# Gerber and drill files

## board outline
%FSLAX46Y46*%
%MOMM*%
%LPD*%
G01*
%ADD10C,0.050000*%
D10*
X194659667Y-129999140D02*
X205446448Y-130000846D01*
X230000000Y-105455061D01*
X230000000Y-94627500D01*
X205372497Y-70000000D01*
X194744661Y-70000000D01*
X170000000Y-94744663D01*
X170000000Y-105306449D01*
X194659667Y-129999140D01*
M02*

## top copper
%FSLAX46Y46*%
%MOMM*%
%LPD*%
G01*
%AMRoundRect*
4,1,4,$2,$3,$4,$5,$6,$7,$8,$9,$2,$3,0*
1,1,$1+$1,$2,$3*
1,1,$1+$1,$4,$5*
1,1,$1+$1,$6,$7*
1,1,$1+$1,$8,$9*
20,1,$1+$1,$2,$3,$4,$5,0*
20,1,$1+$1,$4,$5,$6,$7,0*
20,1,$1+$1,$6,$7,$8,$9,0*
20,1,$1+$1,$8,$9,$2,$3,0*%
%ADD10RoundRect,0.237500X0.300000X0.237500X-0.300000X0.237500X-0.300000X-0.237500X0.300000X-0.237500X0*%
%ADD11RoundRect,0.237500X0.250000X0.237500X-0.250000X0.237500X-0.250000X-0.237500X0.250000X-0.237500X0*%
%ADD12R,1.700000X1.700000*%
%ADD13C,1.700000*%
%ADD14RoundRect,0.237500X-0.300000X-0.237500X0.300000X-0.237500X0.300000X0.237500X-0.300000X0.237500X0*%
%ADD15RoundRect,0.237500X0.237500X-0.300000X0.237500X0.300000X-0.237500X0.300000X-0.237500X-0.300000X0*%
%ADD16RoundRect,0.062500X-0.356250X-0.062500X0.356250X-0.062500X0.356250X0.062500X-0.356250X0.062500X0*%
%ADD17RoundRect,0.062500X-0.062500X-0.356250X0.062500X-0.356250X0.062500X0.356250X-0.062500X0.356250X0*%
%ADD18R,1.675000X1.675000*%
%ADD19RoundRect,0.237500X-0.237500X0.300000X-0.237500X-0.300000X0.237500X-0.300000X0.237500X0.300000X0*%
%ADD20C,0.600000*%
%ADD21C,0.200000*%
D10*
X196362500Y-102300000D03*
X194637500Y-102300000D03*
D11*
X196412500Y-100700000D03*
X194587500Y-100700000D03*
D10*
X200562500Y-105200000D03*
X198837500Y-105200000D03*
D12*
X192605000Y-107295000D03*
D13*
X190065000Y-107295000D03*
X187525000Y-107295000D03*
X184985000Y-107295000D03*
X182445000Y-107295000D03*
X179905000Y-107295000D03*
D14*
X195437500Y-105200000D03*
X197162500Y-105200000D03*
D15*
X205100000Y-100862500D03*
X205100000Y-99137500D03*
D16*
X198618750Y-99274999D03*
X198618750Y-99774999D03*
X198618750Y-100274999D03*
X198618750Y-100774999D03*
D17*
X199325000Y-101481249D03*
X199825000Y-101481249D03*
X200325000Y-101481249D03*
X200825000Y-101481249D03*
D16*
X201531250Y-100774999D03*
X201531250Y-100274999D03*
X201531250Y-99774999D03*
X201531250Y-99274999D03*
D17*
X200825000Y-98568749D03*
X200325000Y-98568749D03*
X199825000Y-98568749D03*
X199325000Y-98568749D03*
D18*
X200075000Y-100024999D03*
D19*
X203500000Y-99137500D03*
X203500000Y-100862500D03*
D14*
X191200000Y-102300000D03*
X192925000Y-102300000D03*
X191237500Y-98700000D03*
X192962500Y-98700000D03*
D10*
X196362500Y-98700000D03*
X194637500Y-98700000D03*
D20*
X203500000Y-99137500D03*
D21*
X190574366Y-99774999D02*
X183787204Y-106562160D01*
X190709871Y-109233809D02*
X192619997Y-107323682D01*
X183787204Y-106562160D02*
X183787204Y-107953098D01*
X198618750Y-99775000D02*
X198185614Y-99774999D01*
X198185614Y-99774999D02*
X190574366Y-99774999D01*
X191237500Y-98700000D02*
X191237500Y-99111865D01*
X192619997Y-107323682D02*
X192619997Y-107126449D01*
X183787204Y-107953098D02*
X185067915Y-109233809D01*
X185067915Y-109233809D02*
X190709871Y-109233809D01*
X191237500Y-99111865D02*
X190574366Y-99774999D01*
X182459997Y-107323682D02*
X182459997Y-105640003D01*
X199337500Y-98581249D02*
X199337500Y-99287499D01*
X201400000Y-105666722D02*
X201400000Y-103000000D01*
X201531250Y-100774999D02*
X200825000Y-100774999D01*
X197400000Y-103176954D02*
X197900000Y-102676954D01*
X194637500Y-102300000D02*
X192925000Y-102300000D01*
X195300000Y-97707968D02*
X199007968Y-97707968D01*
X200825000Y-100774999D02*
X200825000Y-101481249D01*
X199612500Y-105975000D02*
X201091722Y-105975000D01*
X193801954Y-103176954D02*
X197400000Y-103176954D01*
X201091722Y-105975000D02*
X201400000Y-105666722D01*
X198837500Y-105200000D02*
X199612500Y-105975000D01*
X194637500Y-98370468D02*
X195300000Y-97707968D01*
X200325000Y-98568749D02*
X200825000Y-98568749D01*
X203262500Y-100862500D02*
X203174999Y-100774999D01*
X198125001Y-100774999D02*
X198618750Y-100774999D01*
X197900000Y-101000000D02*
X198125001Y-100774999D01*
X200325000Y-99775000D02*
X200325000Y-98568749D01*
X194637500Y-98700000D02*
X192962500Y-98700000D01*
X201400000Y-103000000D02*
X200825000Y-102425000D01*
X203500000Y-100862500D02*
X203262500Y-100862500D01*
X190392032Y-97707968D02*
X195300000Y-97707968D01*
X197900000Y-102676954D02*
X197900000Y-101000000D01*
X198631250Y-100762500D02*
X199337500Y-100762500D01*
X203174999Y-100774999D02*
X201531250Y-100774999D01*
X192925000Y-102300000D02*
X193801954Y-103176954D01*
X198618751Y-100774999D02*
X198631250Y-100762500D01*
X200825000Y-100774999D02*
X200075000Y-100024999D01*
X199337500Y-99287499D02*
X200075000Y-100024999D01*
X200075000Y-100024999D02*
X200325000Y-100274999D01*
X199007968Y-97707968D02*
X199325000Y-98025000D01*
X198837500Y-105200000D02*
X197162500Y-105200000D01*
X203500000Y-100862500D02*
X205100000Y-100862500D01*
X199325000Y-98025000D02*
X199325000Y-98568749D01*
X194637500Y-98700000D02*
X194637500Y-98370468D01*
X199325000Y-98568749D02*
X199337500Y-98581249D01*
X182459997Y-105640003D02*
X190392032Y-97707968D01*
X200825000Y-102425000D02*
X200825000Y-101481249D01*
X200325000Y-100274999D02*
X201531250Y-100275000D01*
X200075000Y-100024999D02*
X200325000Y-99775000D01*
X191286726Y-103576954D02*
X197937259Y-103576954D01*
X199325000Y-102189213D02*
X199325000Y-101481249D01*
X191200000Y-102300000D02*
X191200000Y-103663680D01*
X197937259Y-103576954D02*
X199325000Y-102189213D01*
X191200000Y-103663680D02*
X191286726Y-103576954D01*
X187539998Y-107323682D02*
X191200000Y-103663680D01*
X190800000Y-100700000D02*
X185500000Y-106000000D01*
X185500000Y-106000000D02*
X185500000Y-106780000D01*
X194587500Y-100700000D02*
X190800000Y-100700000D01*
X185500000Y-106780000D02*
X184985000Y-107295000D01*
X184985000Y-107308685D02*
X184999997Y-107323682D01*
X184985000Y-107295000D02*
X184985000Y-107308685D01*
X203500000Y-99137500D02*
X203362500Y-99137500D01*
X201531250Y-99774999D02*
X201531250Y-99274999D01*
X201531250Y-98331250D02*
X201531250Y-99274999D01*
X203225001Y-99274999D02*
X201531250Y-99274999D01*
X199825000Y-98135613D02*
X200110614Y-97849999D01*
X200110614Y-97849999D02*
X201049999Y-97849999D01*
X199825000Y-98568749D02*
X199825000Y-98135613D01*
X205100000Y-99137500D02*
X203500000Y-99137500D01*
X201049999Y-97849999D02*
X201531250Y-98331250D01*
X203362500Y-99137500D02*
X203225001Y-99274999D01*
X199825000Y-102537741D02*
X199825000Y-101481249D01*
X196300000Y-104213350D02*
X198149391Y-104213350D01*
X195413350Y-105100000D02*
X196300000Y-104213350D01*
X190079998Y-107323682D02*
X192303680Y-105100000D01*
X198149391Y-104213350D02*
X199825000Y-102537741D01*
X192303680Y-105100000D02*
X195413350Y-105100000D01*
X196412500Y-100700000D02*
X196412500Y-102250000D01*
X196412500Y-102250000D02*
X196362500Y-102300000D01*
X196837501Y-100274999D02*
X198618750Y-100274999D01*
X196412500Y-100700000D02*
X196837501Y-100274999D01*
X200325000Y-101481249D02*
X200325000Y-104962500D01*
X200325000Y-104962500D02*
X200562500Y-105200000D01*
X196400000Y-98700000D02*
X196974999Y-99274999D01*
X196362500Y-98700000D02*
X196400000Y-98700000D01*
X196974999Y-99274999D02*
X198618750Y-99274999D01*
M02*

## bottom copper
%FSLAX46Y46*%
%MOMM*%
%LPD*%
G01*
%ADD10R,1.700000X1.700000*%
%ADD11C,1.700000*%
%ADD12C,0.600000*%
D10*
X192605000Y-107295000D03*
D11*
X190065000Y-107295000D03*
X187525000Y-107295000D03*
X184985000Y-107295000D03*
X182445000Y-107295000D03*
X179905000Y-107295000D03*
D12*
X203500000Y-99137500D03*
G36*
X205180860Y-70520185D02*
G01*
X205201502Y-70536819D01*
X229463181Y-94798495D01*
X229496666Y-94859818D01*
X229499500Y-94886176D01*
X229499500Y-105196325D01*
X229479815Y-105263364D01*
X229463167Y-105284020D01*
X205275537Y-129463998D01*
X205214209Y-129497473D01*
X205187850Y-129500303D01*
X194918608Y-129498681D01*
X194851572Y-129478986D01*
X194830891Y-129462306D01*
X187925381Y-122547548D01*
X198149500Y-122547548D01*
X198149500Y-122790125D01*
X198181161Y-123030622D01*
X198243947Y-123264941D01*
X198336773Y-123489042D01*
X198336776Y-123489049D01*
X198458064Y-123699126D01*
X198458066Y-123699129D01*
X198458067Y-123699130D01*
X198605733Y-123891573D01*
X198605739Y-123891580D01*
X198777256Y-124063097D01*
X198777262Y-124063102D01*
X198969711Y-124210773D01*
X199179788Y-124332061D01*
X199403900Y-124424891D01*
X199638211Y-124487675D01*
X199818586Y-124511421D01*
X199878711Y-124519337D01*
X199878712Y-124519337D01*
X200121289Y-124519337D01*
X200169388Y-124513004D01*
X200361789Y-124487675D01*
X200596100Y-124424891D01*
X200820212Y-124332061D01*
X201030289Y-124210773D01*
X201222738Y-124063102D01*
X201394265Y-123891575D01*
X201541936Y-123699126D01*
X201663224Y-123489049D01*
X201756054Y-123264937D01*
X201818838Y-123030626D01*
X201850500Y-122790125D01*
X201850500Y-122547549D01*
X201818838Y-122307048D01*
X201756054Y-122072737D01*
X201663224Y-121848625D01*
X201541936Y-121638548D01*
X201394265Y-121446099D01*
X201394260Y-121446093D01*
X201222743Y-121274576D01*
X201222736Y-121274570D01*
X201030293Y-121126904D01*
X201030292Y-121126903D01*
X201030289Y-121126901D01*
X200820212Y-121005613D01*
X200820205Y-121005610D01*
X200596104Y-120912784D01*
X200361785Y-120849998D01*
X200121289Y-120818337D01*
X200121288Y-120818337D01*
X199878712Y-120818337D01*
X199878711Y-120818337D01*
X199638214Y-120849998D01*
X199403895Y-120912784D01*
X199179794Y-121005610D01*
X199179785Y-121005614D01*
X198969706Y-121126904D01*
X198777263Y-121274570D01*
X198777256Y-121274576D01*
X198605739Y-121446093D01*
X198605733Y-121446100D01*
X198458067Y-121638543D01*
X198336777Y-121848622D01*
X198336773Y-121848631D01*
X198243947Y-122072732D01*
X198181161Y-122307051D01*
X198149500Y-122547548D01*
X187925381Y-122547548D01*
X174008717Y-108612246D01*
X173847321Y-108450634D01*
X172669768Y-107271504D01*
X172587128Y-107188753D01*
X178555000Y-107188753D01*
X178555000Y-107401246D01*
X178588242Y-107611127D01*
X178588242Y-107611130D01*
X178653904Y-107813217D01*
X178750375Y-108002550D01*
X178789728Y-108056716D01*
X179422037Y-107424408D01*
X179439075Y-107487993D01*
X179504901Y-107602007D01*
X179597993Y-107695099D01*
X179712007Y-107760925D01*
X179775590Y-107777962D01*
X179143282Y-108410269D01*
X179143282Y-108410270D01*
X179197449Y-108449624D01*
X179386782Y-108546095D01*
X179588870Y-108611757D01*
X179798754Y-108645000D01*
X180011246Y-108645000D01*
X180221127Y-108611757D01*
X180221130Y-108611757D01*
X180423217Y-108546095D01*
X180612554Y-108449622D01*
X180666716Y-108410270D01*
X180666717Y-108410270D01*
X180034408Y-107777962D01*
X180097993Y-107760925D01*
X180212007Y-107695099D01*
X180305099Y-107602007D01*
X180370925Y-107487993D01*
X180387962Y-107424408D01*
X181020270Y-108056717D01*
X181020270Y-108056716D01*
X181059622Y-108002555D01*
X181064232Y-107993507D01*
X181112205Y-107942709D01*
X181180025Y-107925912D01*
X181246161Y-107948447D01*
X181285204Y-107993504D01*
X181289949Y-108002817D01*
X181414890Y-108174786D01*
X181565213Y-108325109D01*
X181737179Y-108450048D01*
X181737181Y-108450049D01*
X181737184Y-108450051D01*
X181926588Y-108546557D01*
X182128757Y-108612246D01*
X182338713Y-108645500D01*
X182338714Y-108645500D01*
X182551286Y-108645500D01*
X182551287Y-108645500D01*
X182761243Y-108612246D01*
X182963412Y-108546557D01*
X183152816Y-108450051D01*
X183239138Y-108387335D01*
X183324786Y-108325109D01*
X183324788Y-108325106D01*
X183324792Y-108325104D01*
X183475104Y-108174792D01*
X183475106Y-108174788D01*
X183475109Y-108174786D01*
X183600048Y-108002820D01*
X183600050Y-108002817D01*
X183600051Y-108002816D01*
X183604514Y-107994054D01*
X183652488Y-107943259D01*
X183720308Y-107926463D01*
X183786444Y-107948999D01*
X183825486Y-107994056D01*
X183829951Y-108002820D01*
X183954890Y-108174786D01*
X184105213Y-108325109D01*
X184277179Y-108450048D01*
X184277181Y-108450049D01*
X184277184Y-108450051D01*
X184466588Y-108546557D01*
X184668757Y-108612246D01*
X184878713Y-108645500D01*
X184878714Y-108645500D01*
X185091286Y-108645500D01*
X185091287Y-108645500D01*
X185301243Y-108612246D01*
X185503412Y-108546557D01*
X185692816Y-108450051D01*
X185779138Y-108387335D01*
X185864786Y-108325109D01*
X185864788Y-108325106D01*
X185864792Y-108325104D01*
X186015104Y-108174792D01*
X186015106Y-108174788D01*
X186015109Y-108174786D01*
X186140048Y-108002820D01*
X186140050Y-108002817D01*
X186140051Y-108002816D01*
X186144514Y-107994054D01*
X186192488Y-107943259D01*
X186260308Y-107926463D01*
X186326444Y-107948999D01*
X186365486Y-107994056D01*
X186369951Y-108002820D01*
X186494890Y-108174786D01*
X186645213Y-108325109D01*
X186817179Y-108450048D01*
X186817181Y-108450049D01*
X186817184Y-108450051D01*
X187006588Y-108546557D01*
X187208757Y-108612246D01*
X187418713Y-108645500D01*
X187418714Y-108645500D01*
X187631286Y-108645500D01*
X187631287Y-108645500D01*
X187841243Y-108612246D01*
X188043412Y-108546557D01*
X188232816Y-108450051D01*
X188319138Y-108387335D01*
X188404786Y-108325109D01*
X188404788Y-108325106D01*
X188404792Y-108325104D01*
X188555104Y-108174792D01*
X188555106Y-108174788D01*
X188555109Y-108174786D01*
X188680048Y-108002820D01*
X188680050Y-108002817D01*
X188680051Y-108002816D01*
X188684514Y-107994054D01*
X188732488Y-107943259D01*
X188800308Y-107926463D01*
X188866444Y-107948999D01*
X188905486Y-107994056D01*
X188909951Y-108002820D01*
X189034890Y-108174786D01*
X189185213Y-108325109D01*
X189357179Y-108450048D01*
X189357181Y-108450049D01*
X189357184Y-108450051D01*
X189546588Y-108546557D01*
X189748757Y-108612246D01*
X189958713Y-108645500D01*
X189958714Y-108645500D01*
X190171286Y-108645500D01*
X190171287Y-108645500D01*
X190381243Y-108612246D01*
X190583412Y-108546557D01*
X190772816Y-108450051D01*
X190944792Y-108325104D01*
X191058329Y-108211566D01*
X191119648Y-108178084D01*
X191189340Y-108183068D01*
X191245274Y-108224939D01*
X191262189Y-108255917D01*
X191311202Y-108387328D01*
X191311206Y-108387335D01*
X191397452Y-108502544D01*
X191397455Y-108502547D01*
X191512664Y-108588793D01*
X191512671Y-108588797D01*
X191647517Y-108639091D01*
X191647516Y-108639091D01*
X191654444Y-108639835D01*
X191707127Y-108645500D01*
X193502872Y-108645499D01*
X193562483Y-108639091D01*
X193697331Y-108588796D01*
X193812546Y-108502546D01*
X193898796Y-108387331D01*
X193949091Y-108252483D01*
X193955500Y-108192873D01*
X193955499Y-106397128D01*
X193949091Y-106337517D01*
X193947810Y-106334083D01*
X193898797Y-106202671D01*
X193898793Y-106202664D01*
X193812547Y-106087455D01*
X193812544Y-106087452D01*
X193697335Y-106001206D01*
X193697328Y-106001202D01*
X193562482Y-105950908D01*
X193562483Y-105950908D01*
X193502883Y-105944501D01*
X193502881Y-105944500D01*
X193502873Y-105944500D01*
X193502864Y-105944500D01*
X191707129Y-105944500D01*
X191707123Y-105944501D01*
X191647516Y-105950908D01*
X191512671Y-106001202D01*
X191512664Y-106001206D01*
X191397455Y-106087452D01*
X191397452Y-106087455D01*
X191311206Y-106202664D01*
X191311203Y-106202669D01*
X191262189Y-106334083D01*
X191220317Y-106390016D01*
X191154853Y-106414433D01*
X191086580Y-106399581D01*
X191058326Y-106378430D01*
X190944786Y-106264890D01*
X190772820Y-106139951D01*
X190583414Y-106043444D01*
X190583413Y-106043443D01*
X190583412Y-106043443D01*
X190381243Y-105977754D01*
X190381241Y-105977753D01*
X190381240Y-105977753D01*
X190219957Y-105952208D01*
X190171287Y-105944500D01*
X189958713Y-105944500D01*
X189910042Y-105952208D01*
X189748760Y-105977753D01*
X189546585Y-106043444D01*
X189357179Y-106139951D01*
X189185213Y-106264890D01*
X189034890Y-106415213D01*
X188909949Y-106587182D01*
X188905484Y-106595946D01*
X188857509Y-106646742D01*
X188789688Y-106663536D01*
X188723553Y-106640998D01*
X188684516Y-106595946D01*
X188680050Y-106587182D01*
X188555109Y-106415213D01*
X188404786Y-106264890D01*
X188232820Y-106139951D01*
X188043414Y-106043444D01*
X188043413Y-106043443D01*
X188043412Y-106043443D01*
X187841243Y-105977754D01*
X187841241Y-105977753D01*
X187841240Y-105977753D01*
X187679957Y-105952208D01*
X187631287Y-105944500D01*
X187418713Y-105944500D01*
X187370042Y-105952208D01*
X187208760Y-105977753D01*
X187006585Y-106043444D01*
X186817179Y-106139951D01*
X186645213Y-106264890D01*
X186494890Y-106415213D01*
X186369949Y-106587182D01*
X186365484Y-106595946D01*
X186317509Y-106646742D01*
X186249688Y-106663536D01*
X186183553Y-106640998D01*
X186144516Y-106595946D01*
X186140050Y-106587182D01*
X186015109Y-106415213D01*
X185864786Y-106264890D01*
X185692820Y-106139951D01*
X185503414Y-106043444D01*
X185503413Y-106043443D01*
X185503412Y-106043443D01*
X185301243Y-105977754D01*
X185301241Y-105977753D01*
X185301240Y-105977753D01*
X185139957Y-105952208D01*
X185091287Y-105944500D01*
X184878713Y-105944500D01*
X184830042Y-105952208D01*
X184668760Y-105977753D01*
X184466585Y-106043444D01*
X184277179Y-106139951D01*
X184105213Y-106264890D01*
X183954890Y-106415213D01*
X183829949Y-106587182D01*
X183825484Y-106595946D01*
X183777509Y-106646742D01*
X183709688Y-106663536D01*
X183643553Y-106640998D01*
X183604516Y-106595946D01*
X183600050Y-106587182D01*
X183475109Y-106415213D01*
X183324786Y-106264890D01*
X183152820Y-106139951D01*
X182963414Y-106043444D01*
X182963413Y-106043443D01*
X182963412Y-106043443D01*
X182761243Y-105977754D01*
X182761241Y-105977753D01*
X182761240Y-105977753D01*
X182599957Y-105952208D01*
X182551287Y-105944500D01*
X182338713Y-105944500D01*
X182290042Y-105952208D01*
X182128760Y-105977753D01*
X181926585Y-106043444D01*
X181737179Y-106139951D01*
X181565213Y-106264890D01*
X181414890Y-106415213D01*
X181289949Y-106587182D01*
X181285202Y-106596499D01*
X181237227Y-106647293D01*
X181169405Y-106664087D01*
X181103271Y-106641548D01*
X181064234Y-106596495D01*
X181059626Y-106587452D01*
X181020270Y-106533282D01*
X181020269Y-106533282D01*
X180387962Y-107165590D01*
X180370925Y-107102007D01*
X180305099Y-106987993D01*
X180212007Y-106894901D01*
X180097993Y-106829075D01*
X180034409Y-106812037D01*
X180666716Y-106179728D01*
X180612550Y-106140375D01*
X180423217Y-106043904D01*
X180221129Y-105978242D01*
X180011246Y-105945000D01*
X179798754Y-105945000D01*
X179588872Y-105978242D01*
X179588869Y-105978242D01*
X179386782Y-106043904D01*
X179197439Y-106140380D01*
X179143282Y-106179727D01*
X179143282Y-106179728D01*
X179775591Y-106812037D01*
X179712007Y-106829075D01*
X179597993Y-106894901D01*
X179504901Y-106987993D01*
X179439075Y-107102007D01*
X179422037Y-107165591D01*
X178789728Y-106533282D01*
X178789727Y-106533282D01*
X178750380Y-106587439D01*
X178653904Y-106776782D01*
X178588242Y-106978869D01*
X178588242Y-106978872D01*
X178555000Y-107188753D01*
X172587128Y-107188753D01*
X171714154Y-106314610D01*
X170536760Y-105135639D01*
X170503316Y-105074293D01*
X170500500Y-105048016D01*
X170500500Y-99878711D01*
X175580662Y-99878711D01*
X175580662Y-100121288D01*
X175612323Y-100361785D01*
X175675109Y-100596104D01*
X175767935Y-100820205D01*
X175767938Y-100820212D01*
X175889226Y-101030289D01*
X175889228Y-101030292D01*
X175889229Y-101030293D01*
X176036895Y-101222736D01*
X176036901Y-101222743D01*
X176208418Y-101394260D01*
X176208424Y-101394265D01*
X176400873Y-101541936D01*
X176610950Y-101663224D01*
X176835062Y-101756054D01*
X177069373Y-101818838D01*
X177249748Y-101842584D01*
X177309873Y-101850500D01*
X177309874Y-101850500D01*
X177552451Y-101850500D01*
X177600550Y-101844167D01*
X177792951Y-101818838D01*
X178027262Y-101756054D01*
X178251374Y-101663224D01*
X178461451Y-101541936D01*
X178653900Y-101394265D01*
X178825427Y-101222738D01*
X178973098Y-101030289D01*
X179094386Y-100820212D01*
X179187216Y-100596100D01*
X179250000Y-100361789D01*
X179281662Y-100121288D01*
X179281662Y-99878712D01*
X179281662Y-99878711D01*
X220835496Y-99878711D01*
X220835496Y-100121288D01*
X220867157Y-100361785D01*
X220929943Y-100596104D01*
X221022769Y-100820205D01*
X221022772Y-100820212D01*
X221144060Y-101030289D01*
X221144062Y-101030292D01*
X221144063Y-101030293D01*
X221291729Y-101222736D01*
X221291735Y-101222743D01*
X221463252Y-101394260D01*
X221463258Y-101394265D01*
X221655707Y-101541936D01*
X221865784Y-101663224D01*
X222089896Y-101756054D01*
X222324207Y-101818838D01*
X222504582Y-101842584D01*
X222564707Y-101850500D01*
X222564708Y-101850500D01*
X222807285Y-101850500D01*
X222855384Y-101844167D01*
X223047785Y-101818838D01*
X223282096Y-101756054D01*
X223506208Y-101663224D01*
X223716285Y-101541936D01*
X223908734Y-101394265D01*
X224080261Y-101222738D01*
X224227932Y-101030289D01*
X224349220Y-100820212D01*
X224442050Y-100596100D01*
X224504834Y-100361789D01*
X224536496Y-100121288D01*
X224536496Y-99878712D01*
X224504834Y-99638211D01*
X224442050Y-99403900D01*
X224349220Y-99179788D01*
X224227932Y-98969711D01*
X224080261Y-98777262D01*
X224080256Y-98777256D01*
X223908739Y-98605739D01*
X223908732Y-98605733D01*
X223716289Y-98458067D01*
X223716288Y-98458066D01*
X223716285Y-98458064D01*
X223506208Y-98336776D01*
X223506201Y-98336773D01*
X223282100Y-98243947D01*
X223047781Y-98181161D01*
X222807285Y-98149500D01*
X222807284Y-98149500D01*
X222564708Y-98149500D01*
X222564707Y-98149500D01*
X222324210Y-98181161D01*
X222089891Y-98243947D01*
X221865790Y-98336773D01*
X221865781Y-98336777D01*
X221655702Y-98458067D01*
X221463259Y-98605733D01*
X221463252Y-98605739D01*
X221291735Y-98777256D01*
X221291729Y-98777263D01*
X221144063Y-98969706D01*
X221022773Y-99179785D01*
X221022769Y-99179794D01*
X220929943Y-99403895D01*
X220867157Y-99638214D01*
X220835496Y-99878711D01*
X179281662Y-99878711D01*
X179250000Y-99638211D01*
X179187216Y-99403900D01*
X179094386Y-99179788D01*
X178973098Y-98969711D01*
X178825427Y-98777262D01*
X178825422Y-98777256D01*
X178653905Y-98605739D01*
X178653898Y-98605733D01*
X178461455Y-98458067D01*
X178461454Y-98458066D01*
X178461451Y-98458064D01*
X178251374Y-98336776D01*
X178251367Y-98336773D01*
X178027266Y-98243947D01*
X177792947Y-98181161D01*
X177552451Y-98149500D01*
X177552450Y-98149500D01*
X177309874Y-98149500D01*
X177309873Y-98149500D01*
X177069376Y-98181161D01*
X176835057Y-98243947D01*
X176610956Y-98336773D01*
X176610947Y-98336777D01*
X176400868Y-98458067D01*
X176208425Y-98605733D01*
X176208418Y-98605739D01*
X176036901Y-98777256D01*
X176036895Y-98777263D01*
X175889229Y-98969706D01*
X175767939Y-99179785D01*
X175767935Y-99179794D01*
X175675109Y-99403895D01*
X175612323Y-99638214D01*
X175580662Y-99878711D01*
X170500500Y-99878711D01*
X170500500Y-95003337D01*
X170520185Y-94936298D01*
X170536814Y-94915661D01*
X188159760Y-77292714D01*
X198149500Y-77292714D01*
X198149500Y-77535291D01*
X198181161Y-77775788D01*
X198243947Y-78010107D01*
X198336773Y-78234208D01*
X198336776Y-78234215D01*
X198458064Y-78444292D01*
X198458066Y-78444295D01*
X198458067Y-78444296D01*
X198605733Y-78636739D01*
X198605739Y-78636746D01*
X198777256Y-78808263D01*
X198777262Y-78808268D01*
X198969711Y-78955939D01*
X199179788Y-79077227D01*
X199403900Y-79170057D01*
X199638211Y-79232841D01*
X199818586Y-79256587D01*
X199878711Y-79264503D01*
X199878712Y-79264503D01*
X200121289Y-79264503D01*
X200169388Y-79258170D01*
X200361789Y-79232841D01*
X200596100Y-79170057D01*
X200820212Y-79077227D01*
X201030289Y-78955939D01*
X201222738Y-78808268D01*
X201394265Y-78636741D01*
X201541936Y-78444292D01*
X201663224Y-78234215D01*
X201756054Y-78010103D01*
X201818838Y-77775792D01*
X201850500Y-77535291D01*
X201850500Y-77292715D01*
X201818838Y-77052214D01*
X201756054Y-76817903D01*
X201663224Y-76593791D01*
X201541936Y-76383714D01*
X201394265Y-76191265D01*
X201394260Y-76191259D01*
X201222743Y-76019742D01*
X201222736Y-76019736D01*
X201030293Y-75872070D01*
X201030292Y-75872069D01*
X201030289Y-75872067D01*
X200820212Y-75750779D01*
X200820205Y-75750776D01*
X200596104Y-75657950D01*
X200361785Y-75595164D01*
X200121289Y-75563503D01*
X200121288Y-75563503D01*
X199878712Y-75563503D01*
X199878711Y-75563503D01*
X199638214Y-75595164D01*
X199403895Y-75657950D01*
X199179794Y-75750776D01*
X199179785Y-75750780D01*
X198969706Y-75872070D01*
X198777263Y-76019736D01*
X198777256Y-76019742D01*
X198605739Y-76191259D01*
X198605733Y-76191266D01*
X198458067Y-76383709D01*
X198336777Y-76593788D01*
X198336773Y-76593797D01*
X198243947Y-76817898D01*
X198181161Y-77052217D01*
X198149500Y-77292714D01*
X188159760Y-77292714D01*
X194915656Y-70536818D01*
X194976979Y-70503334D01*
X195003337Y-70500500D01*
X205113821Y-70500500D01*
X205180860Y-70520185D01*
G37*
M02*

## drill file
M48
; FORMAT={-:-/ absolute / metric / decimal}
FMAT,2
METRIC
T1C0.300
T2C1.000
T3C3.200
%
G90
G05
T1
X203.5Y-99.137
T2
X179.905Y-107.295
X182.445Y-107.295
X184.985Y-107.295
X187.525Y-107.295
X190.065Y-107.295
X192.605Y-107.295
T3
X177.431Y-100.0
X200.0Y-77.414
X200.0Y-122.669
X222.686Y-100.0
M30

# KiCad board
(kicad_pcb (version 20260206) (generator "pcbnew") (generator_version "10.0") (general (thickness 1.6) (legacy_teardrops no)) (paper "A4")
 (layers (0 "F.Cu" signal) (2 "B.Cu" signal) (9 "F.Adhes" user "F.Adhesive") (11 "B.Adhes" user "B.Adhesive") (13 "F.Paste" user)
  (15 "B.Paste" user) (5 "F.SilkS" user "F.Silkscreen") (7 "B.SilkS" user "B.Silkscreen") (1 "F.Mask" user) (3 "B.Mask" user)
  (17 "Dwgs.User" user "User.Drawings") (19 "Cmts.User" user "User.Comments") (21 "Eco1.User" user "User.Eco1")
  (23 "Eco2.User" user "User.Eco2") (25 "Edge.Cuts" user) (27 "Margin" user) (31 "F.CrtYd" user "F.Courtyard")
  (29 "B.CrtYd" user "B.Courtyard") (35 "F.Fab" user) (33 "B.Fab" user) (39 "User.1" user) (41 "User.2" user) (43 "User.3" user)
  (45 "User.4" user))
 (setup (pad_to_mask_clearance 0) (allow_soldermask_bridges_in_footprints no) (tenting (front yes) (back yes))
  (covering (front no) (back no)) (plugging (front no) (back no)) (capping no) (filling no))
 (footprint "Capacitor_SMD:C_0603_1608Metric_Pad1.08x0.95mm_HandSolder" (layer "F.Cu") (at 195.5 102.3 180)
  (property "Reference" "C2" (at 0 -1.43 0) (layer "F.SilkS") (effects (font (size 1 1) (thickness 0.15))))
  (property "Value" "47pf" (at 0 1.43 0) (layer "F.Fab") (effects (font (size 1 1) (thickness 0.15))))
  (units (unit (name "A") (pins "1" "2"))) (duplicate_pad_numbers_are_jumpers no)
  (pad "1" smd roundrect (at -0.8625 0 180) (size 1.075 0.95) (layers "F.Cu" "F.Mask" "F.Paste") (roundrect_rratio 0.25)
   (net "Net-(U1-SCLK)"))
  (pad "2" smd roundrect (at 0.8625 0 180) (size 1.075 0.95) (layers "F.Cu" "F.Mask" "F.Paste") (roundrect_rratio 0.25) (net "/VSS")))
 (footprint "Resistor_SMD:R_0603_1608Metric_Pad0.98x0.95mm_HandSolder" (layer "F.Cu") (at 195.5 100.7 180)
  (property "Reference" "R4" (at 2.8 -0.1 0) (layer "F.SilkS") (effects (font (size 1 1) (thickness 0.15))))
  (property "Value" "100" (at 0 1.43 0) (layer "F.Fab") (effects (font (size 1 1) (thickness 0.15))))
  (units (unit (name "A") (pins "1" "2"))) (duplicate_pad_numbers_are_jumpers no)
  (pad "1" smd roundrect (at -0.9125 0 180) (size 0.975 0.95) (layers "F.Cu" "F.Mask" "F.Paste") (roundrect_rratio 0.25)
   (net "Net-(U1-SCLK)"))
  (pad "2" smd roundrect (at 0.9125 0 180) (size 0.975 0.95) (layers "F.Cu" "F.Mask" "F.Paste") (roundrect_rratio 0.25) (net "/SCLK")))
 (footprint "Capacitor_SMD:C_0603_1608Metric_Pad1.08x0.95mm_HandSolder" (layer "F.Cu") (at 199.7 105.2 180)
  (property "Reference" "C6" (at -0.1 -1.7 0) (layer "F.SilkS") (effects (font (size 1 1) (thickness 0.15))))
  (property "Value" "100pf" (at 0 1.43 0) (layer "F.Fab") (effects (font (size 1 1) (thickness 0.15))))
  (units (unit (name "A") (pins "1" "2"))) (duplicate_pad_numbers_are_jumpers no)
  (pad "1" smd roundrect (at -0.8625 0 180) (size 1.075 0.95) (layers "F.Cu" "F.Mask" "F.Paste") (roundrect_rratio 0.25)
   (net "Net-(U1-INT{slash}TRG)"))
  (pad "2" smd roundrect (at 0.8625 0 180) (size 1.075 0.95) (layers "F.Cu" "F.Mask" "F.Paste") (roundrect_rratio 0.25) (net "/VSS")))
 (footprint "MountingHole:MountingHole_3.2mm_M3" (layer "F.Cu") (at 200 77.414003 45)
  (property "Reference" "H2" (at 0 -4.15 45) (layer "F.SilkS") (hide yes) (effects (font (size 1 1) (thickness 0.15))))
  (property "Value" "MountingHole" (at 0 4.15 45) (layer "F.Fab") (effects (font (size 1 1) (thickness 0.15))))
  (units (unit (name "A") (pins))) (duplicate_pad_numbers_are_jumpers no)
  (pad "" np_thru_hole circle (at 0 0 45) (size 3.2 3.2) (drill 3.2) (layers "*.Cu" "*.Mask")))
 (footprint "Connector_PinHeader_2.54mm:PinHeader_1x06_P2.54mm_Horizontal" (layer "F.Cu") (at 192.605 107.295 -90)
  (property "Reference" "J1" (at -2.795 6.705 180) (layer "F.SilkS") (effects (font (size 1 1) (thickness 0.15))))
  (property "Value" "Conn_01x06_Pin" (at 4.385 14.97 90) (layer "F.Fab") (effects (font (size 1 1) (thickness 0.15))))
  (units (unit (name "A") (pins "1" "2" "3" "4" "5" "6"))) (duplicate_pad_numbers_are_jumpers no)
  (pad "1" thru_hole rect (at 0 0 270) (size 1.7 1.7) (drill 1) (layers "*.Cu" "*.Mask") (remove_unused_layers no) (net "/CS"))
  (pad "2" thru_hole circle (at 0 2.54 270) (size 1.7 1.7) (drill 1) (layers "*.Cu" "*.Mask") (remove_unused_layers no) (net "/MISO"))
  (pad "3" thru_hole circle (at 0 5.08 270) (size 1.7 1.7) (drill 1) (layers "*.Cu" "*.Mask") (remove_unused_layers no) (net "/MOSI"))
  (pad "4" thru_hole circle (at 0 7.62 270) (size 1.7 1.7) (drill 1) (layers "*.Cu" "*.Mask") (remove_unused_layers no) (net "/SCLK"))
  (pad "5" thru_hole circle (at 0 10.16 270) (size 1.7 1.7) (drill 1) (layers "*.Cu" "*.Mask") (remove_unused_layers no) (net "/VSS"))
  (pad "6" thru_hole circle (at 0 12.7 270) (size 1.7 1.7) (drill 1) (layers "*.Cu" "*.Mask") (remove_unused_layers no) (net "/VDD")))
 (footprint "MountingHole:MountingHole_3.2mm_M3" (layer "F.Cu") (at 200 122.668837 45)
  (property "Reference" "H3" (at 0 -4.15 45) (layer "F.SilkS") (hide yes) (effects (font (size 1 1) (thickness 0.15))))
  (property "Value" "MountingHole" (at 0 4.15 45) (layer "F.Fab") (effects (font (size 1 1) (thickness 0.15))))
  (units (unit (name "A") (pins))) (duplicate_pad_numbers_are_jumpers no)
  (pad "" np_thru_hole circle (at 0 0 45) (size 3.2 3.2) (drill 3.2) (layers "*.Cu" "*.Mask")))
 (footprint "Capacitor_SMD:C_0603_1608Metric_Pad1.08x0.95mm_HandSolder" (layer "F.Cu") (at 196.3 105.2)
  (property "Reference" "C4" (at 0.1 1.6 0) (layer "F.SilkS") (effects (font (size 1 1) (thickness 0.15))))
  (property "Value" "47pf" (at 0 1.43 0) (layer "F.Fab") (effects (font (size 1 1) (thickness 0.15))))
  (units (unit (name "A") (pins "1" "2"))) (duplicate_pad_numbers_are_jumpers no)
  (pad "1" smd roundrect (at -0.8625 0) (size 1.075 0.95) (layers "F.Cu" "F.Mask" "F.Paste") (roundrect_rratio 0.25) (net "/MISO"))
  (pad "2" smd roundrect (at 0.8625 0) (size 1.075 0.95) (layers "F.Cu" "F.Mask" "F.Paste") (roundrect_rratio 0.25) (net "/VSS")))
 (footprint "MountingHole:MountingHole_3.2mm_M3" (layer "F.Cu") (at 222.685996 100 45)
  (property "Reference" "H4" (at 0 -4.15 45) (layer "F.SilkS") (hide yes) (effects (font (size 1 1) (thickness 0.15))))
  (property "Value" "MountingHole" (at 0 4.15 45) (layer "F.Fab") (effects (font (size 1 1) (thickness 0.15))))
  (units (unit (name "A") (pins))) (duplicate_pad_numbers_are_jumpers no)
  (pad "" np_thru_hole circle (at 0 0 45) (size 3.2 3.2) (drill 3.2) (layers "*.Cu" "*.Mask")))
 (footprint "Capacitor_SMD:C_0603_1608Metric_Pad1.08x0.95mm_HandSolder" (layer "F.Cu") (at 205.1 100 90)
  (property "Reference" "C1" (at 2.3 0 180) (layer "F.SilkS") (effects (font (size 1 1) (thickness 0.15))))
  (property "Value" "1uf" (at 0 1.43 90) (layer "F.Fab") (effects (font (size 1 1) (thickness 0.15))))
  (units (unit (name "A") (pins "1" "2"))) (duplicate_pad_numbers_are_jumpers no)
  (pad "1" smd roundrect (at -0.8625 0 90) (size 1.075 0.95) (layers "F.Cu" "F.Mask" "F.Paste") (roundrect_rratio 0.25) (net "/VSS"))
  (pad "2" smd roundrect (at 0.8625 0 90) (size 1.075 0.95) (layers "F.Cu" "F.Mask" "F.Paste") (roundrect_rratio 0.25) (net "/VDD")))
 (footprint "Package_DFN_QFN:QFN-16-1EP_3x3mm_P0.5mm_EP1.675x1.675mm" (layer "F.Cu") (at 200.075 100.024999)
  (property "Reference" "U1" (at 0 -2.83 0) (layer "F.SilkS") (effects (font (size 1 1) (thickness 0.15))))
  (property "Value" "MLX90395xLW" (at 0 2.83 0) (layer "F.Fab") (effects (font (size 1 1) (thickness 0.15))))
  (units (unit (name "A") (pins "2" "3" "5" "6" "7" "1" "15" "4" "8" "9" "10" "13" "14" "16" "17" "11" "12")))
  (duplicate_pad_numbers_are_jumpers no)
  (pad "" smd roundrect (at 0 0) (size 1.35 1.35) (layers "F.Paste") (roundrect_rratio 0.185185))
  (pad "1" smd roundrect (at -1.45625 -0.75) (size 0.8375 0.25) (layers "F.Cu" "F.Mask" "F.Paste") (roundrect_rratio 0.25)
   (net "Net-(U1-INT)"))
  (pad "2" smd roundrect (at -1.45625 -0.25) (size 0.8375 0.25) (layers "F.Cu" "F.Mask" "F.Paste") (roundrect_rratio 0.25) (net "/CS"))
  (pad "3" smd roundrect (at -1.45625 0.25) (size 0.8375 0.25) (layers "F.Cu" "F.Mask" "F.Paste") (roundrect_rratio 0.25)
   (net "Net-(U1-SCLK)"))
  (pad "4" smd roundrect (at -1.45625 0.75) (size 0.8375 0.25) (layers "F.Cu" "F.Mask" "F.Paste") (roundrect_rratio 0.25) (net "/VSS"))
  (pad "5" smd roundrect (at -0.75 1.45625) (size 0.25 0.8375) (layers "F.Cu" "F.Mask" "F.Paste") (roundrect_rratio 0.25) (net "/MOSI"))
  (pad "6" smd roundrect (at -0.25 1.45625) (size 0.25 0.8375) (layers "F.Cu" "F.Mask" "F.Paste") (roundrect_rratio 0.25) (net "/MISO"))
  (pad "7" smd roundrect (at 0.25 1.45625) (size 0.25 0.8375) (layers "F.Cu" "F.Mask" "F.Paste") (roundrect_rratio 0.25)
   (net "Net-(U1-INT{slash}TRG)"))
  (pad "8" smd roundrect (at 0.75 1.45625) (size 0.25 0.8375) (layers "F.Cu" "F.Mask" "F.Paste") (roundrect_rratio 0.25) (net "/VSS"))
  (pad "9" smd roundrect (at 1.45625 0.75) (size 0.8375 0.25) (layers "F.Cu" "F.Mask" "F.Paste") (roundrect_rratio 0.25) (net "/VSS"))
  (pad "10" smd roundrect (at 1.45625 0.25) (size 0.8375 0.25) (layers "F.Cu" "F.Mask" "F.Paste") (roundrect_rratio 0.25) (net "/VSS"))
  (pad "11" smd roundrect (at 1.45625 -0.25) (size 0.8375 0.25) (layers "F.Cu" "F.Mask" "F.Paste") (roundrect_rratio 0.25) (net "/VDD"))
  (pad "12" smd roundrect (at 1.45625 -0.75) (size 0.8375 0.25) (layers "F.Cu" "F.Mask" "F.Paste") (roundrect_rratio 0.25) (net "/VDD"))
  (pad "13" smd roundrect (at 0.75 -1.45625) (size 0.25 0.8375) (layers "F.Cu" "F.Mask" "F.Paste") (roundrect_rratio 0.25) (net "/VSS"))
  (pad "14" smd roundrect (at 0.25 -1.45625) (size 0.25 0.8375) (layers "F.Cu" "F.Mask" "F.Paste") (roundrect_rratio 0.25) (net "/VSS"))
  (pad "15" smd roundrect (at -0.25 -1.45625) (size 0.25 0.8375) (layers "F.Cu" "F.Mask" "F.Paste") (roundrect_rratio 0.25) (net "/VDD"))
  (pad "16" smd roundrect (at -0.75 -1.45625) (size 0.25 0.8375) (layers "F.Cu" "F.Mask" "F.Paste") (roundrect_rratio 0.25) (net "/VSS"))
  (pad "17" smd rect (at 0 0) (size 1.675 1.675) (layers "F.Cu" "F.Mask") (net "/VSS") (zone_connect 2)))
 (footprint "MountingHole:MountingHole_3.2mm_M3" (layer "F.Cu") (at 177.431162 100 45)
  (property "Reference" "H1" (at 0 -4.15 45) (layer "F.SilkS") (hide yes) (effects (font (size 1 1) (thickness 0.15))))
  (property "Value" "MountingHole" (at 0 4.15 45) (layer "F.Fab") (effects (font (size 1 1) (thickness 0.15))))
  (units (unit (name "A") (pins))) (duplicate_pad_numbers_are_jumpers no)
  (pad "" np_thru_hole circle (at 0 0 45) (size 3.2 3.2) (drill 3.2) (layers "*.Cu" "*.Mask")))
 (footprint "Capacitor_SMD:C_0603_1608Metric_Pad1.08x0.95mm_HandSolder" (layer "F.Cu") (at 203.5 100 -90)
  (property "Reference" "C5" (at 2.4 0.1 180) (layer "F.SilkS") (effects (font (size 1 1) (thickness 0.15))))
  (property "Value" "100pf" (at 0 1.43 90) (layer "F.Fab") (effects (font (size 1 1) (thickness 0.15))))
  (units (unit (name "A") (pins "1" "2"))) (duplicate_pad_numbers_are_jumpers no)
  (pad "1" smd roundrect (at -0.8625 0 270) (size 1.075 0.95) (layers "F.Cu" "F.Mask" "F.Paste") (roundrect_rratio 0.25) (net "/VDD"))
  (pad "2" smd roundrect (at 0.8625 0 270) (size 1.075 0.95) (layers "F.Cu" "F.Mask" "F.Paste") (roundrect_rratio 0.25) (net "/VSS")))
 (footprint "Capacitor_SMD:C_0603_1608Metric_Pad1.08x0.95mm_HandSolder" (layer "F.Cu") (at 192.0625 102.3)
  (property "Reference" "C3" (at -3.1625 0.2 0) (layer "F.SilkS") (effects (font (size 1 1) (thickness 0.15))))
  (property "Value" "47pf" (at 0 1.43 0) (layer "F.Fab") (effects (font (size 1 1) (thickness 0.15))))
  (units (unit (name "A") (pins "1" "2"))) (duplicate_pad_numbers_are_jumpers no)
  (pad "1" smd roundrect (at -0.8625 0) (size 1.075 0.95) (layers "F.Cu" "F.Mask" "F.Paste") (roundrect_rratio 0.25) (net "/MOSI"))
  (pad "2" smd roundrect (at 0.8625 0) (size 1.075 0.95) (layers "F.Cu" "F.Mask" "F.Paste") (roundrect_rratio 0.25) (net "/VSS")))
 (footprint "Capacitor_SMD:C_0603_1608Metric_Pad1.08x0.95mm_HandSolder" (layer "F.Cu") (at 192.1 98.7)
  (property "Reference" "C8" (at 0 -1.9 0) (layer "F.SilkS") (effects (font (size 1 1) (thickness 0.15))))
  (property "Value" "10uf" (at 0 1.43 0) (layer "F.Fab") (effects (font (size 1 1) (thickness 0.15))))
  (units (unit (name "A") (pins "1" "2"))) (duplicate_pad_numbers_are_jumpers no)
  (pad "1" smd roundrect (at -0.8625 0) (size 1.075 0.95) (layers "F.Cu" "F.Mask" "F.Paste") (roundrect_rratio 0.25) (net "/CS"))
  (pad "2" smd roundrect (at 0.8625 0) (size 1.075 0.95) (layers "F.Cu" "F.Mask" "F.Paste") (roundrect_rratio 0.25) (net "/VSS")))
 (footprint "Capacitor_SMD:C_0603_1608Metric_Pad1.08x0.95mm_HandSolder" (layer "F.Cu") (at 195.5 98.7 180)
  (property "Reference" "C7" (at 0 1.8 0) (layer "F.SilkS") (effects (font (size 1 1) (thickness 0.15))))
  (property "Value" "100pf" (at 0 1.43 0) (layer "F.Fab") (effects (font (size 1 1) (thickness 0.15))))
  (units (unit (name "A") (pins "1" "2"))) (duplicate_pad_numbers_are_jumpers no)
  (pad "1" smd roundrect (at -0.8625 0 180) (size 1.075 0.95) (layers "F.Cu" "F.Mask" "F.Paste") (roundrect_rratio 0.25)
   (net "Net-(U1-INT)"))
  (pad "2" smd roundrect (at 0.8625 0 180) (size 1.075 0.95) (layers "F.Cu" "F.Mask" "F.Paste") (roundrect_rratio 0.25) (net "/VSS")))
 (gr_poly
  (pts (xy 194.659667 129.99914) (xy 205.446448 130.000846) (xy 230 105.455061) (xy 230 94.6275) (xy 205.372497 70) (xy 194.744661 70)
   (xy 170 94.744663) (xy 170 105.306449))
  (stroke (width 0.05) (type solid)) (fill no) (layer "Edge.Cuts"))
 (segment (start 190.574366 99.774999) (end 183.787204 106.56216) (width 0.2) (layer "F.Cu") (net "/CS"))
 (segment (start 190.709871 109.233809) (end 192.619997 107.323682) (width 0.2) (layer "F.Cu") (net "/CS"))
 (segment (start 183.787204 106.56216) (end 183.787204 107.953098) (width 0.2) (layer "F.Cu") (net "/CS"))
 (segment (start 198.61875 99.775) (end 198.185614 99.774999) (width 0.2) (layer "F.Cu") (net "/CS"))
 (segment (start 198.185614 99.774999) (end 190.574366 99.774999) (width 0.2) (layer "F.Cu") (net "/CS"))
 (segment (start 191.2375 98.7) (end 191.2375 99.111865) (width 0.2) (layer "F.Cu") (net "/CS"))
 (segment (start 192.619997 107.323682) (end 192.619997 107.126449) (width 0.2) (layer "F.Cu") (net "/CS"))
 (segment (start 183.787204 107.953098) (end 185.067915 109.233809) (width 0.2) (layer "F.Cu") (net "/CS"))
 (segment (start 185.067915 109.233809) (end 190.709871 109.233809) (width 0.2) (layer "F.Cu") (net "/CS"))
 (segment (start 191.2375 99.111865) (end 190.574366 99.774999) (width 0.2) (layer "F.Cu") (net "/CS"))
 (segment (start 182.459997 107.323682) (end 182.459997 105.640003) (width 0.2) (layer "F.Cu") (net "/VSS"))
 (segment (start 199.3375 98.581249) (end 199.3375 99.287499) (width 0.2) (layer "F.Cu") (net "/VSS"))
 (segment (start 201.4 105.666722) (end 201.4 103) (width 0.2) (layer "F.Cu") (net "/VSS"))
 (segment (start 201.53125 100.774999) (end 200.825 100.774999) (width 0.2) (layer "F.Cu") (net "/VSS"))
 (segment (start 197.4 103.176954) (end 197.9 102.676954) (width 0.2) (layer "F.Cu") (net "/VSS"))
 (segment (start 194.6375 102.3) (end 192.925 102.3) (width 0.2) (layer "F.Cu") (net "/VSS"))
 (segment (start 195.3 97.707968) (end 199.007968 97.707968) (width 0.2) (layer "F.Cu") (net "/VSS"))
 (segment (start 200.825 100.774999) (end 200.825 101.481249) (width 0.2) (layer "F.Cu") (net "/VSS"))
 (segment (start 199.6125 105.975) (end 201.091722 105.975) (width 0.2) (layer "F.Cu") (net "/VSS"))
 (segment (start 193.801954 103.176954) (end 197.4 103.176954) (width 0.2) (layer "F.Cu") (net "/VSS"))
 (segment (start 201.091722 105.975) (end 201.4 105.666722) (width 0.2) (layer "F.Cu") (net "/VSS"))
 (segment (start 198.8375 105.2) (end 199.6125 105.975) (width 0.2) (layer "F.Cu") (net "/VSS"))
 (segment (start 194.6375 98.370468) (end 195.3 97.707968) (width 0.2) (layer "F.Cu") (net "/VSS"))
 (segment (start 200.325 98.568749) (end 200.825 98.568749) (width 0.2) (layer "F.Cu") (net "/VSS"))
 (segment (start 203.2625 100.8625) (end 203.174999 100.774999) (width 0.2) (layer "F.Cu") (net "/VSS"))
 (segment (start 198.125001 100.774999) (end 198.61875 100.774999) (width 0.2) (layer "F.Cu") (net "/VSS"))
 (segment (start 197.9 101) (end 198.125001 100.774999) (width 0.2) (layer "F.Cu") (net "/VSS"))
 (segment (start 200.325 99.775) (end 200.325 98.568749) (width 0.2) (layer "F.Cu") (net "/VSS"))
 (segment (start 194.6375 98.7) (end 192.9625 98.7) (width 0.2) (layer "F.Cu") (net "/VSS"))
 (segment (start 201.4 103) (end 200.825 102.425) (width 0.2) (layer "F.Cu") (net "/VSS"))
 (segment (start 203.5 100.8625) (end 203.2625 100.8625) (width 0.2) (layer "F.Cu") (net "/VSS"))
 (segment (start 190.392032 97.707968) (end 195.3 97.707968) (width 0.2) (layer "F.Cu") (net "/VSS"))
 (segment (start 197.9 102.676954) (end 197.9 101) (width 0.2) (layer "F.Cu") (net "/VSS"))
 (segment (start 198.63125 100.7625) (end 199.3375 100.7625) (width 0.2) (layer "F.Cu") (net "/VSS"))
 (segment (start 203.174999 100.774999) (end 201.53125 100.774999) (width 0.2) (layer "F.Cu") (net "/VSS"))
 (segment (start 192.925 102.3) (end 193.801954 103.176954) (width 0.2) (layer "F.Cu") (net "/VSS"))
 (segment (start 198.618751 100.774999) (end 198.63125 100.7625) (width 0.2) (layer "F.Cu") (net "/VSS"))
 (segment (start 200.825 100.774999) (end 200.075 100.024999) (width 0.2) (layer "F.Cu") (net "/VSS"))
 (segment (start 199.3375 99.287499) (end 200.075 100.024999) (width 0.2) (layer "F.Cu") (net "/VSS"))
 (segment (start 200.075 100.024999) (end 200.325 100.274999) (width 0.2) (layer "F.Cu") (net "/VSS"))
 (segment (start 199.007968 97.707968) (end 199.325 98.025) (width 0.2) (layer "F.Cu") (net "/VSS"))
 (segment (start 198.8375 105.2) (end 197.1625 105.2) (width 0.2) (layer "F.Cu") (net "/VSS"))
 (segment (start 203.5 100.8625) (end 205.1 100.8625) (width 0.2) (layer "F.Cu") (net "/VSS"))
 (segment (start 199.325 98.025) (end 199.325 98.568749) (width 0.2) (layer "F.Cu") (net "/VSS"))
 (segment (start 194.6375 98.7) (end 194.6375 98.370468) (width 0.2) (layer "F.Cu") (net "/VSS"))
 (segment (start 199.325 98.568749) (end 199.3375 98.581249) (width 0.2) (layer "F.Cu") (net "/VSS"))
 (segment (start 182.459997 105.640003) (end 190.392032 97.707968) (width 0.2) (layer "F.Cu") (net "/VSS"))
 (segment (start 200.825 102.425) (end 200.825 101.481249) (width 0.2) (layer "F.Cu") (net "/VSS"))
 (segment (start 200.325 100.274999) (end 201.53125 100.275) (width 0.2) (layer "F.Cu") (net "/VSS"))
 (segment (start 200.075 100.024999) (end 200.325 99.775) (width 0.2) (layer "F.Cu") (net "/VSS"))
 (segment (start 191.286726 103.576954) (end 197.937259 103.576954) (width 0.2) (layer "F.Cu") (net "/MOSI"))
 (segment (start 199.325 102.189213) (end 199.325 101.481249) (width 0.2) (layer "F.Cu") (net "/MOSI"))
 (segment (start 191.2 102.3) (end 191.2 103.66368) (width 0.2) (layer "F.Cu") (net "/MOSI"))
 (segment (start 197.937259 103.576954) (end 199.325 102.189213) (width 0.2) (layer "F.Cu") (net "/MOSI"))
 (segment (start 191.2 103.66368) (end 191.286726 103.576954) (width 0.2) (layer "F.Cu") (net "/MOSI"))
 (segment (start 187.539998 107.323682) (end 191.2 103.66368) (width 0.2) (layer "F.Cu") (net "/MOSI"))
 (segment (start 190.8 100.7) (end 185.5 106) (width 0.2) (layer "F.Cu") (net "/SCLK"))
 (segment (start 185.5 106) (end 185.5 106.78) (width 0.2) (layer "F.Cu") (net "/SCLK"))
 (segment (start 194.5875 100.7) (end 190.8 100.7) (width 0.2) (layer "F.Cu") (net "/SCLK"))
 (segment (start 185.5 106.78) (end 184.985 107.295) (width 0.2) (layer "F.Cu") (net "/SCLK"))
 (segment (start 184.985 107.308685) (end 184.999997 107.323682) (width 0.2) (layer "F.Cu") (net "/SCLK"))
 (segment (start 184.985 107.295) (end 184.985 107.308685) (width 0.2) (layer "F.Cu") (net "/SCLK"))
 (segment (start 203.5 99.1375) (end 203.3625 99.1375) (width 0.2) (layer "F.Cu") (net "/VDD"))
 (segment (start 201.53125 99.774999) (end 201.53125 99.274999) (width 0.2) (layer "F.Cu") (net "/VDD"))
 (segment (start 201.53125 98.33125) (end 201.53125 99.274999) (width 0.2) (layer "F.Cu") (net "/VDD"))
 (segment (start 203.225001 99.274999) (end 201.53125 99.274999) (width 0.2) (layer "F.Cu") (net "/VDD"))
 (segment (start 199.825 98.135613) (end 200.110614 97.849999) (width 0.2) (layer "F.Cu") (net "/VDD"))
 (segment (start 200.110614 97.849999) (end 201.049999 97.849999) (width 0.2) (layer "F.Cu") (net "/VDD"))
 (segment (start 199.825 98.568749) (end 199.825 98.135613) (width 0.2) (layer "F.Cu") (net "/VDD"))
 (segment (start 205.1 99.1375) (end 203.5 99.1375) (width 0.2) (layer "F.Cu") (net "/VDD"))
 (segment (start 201.049999 97.849999) (end 201.53125 98.33125) (width 0.2) (layer "F.Cu") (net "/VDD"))
 (segment (start 203.3625 99.1375) (end 203.225001 99.274999) (width 0.2) (layer "F.Cu") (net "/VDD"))
 (via (at 203.5 99.1375) (size 0.6) (drill 0.3) (layers "F.Cu" "B.Cu") (free yes) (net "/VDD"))
 (segment (start 199.825 102.537741) (end 199.825 101.481249) (width 0.2) (layer "F.Cu") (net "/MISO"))
 (segment (start 196.3 104.21335) (end 198.149391 104.21335) (width 0.2) (layer "F.Cu") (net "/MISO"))
 (segment (start 195.41335 105.1) (end 196.3 104.21335) (width 0.2) (layer "F.Cu") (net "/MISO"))
 (segment (start 190.079998 107.323682) (end 192.30368 105.1) (width 0.2) (layer "F.Cu") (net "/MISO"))
 (segment (start 198.149391 104.21335) (end 199.825 102.537741) (width 0.2) (layer "F.Cu") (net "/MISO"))
 (segment (start 192.30368 105.1) (end 195.41335 105.1) (width 0.2) (layer "F.Cu") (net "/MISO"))
 (segment (start 196.4125 100.7) (end 196.4125 102.25) (width 0.2) (layer "F.Cu") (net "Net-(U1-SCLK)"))
 (segment (start 196.4125 102.25) (end 196.3625 102.3) (width 0.2) (layer "F.Cu") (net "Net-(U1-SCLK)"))
 (segment (start 196.837501 100.274999) (end 198.61875 100.274999) (width 0.2) (layer "F.Cu") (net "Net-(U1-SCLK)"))
 (segment (start 196.4125 100.7) (end 196.837501 100.274999) (width 0.2) (layer "F.Cu") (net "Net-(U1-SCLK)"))
 (segment (start 200.325 101.481249) (end 200.325 104.9625) (width 0.2) (layer "F.Cu") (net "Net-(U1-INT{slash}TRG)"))
 (segment (start 200.325 104.9625) (end 200.5625 105.2) (width 0.2) (layer "F.Cu") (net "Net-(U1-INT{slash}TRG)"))
 (segment (start 196.4 98.7) (end 196.974999 99.274999) (width 0.2) (layer "F.Cu") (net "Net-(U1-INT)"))
 (segment (start 196.3625 98.7) (end 196.4 98.7) (width 0.2) (layer "F.Cu") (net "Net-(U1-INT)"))
 (segment (start 196.974999 99.274999) (end 198.61875 99.274999) (width 0.2) (layer "F.Cu") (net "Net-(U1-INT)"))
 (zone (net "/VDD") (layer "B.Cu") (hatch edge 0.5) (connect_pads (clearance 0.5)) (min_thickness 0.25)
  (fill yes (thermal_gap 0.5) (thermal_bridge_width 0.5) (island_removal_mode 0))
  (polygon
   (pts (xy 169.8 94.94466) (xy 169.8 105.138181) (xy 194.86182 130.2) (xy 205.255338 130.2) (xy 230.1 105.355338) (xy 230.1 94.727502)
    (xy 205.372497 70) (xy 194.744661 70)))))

